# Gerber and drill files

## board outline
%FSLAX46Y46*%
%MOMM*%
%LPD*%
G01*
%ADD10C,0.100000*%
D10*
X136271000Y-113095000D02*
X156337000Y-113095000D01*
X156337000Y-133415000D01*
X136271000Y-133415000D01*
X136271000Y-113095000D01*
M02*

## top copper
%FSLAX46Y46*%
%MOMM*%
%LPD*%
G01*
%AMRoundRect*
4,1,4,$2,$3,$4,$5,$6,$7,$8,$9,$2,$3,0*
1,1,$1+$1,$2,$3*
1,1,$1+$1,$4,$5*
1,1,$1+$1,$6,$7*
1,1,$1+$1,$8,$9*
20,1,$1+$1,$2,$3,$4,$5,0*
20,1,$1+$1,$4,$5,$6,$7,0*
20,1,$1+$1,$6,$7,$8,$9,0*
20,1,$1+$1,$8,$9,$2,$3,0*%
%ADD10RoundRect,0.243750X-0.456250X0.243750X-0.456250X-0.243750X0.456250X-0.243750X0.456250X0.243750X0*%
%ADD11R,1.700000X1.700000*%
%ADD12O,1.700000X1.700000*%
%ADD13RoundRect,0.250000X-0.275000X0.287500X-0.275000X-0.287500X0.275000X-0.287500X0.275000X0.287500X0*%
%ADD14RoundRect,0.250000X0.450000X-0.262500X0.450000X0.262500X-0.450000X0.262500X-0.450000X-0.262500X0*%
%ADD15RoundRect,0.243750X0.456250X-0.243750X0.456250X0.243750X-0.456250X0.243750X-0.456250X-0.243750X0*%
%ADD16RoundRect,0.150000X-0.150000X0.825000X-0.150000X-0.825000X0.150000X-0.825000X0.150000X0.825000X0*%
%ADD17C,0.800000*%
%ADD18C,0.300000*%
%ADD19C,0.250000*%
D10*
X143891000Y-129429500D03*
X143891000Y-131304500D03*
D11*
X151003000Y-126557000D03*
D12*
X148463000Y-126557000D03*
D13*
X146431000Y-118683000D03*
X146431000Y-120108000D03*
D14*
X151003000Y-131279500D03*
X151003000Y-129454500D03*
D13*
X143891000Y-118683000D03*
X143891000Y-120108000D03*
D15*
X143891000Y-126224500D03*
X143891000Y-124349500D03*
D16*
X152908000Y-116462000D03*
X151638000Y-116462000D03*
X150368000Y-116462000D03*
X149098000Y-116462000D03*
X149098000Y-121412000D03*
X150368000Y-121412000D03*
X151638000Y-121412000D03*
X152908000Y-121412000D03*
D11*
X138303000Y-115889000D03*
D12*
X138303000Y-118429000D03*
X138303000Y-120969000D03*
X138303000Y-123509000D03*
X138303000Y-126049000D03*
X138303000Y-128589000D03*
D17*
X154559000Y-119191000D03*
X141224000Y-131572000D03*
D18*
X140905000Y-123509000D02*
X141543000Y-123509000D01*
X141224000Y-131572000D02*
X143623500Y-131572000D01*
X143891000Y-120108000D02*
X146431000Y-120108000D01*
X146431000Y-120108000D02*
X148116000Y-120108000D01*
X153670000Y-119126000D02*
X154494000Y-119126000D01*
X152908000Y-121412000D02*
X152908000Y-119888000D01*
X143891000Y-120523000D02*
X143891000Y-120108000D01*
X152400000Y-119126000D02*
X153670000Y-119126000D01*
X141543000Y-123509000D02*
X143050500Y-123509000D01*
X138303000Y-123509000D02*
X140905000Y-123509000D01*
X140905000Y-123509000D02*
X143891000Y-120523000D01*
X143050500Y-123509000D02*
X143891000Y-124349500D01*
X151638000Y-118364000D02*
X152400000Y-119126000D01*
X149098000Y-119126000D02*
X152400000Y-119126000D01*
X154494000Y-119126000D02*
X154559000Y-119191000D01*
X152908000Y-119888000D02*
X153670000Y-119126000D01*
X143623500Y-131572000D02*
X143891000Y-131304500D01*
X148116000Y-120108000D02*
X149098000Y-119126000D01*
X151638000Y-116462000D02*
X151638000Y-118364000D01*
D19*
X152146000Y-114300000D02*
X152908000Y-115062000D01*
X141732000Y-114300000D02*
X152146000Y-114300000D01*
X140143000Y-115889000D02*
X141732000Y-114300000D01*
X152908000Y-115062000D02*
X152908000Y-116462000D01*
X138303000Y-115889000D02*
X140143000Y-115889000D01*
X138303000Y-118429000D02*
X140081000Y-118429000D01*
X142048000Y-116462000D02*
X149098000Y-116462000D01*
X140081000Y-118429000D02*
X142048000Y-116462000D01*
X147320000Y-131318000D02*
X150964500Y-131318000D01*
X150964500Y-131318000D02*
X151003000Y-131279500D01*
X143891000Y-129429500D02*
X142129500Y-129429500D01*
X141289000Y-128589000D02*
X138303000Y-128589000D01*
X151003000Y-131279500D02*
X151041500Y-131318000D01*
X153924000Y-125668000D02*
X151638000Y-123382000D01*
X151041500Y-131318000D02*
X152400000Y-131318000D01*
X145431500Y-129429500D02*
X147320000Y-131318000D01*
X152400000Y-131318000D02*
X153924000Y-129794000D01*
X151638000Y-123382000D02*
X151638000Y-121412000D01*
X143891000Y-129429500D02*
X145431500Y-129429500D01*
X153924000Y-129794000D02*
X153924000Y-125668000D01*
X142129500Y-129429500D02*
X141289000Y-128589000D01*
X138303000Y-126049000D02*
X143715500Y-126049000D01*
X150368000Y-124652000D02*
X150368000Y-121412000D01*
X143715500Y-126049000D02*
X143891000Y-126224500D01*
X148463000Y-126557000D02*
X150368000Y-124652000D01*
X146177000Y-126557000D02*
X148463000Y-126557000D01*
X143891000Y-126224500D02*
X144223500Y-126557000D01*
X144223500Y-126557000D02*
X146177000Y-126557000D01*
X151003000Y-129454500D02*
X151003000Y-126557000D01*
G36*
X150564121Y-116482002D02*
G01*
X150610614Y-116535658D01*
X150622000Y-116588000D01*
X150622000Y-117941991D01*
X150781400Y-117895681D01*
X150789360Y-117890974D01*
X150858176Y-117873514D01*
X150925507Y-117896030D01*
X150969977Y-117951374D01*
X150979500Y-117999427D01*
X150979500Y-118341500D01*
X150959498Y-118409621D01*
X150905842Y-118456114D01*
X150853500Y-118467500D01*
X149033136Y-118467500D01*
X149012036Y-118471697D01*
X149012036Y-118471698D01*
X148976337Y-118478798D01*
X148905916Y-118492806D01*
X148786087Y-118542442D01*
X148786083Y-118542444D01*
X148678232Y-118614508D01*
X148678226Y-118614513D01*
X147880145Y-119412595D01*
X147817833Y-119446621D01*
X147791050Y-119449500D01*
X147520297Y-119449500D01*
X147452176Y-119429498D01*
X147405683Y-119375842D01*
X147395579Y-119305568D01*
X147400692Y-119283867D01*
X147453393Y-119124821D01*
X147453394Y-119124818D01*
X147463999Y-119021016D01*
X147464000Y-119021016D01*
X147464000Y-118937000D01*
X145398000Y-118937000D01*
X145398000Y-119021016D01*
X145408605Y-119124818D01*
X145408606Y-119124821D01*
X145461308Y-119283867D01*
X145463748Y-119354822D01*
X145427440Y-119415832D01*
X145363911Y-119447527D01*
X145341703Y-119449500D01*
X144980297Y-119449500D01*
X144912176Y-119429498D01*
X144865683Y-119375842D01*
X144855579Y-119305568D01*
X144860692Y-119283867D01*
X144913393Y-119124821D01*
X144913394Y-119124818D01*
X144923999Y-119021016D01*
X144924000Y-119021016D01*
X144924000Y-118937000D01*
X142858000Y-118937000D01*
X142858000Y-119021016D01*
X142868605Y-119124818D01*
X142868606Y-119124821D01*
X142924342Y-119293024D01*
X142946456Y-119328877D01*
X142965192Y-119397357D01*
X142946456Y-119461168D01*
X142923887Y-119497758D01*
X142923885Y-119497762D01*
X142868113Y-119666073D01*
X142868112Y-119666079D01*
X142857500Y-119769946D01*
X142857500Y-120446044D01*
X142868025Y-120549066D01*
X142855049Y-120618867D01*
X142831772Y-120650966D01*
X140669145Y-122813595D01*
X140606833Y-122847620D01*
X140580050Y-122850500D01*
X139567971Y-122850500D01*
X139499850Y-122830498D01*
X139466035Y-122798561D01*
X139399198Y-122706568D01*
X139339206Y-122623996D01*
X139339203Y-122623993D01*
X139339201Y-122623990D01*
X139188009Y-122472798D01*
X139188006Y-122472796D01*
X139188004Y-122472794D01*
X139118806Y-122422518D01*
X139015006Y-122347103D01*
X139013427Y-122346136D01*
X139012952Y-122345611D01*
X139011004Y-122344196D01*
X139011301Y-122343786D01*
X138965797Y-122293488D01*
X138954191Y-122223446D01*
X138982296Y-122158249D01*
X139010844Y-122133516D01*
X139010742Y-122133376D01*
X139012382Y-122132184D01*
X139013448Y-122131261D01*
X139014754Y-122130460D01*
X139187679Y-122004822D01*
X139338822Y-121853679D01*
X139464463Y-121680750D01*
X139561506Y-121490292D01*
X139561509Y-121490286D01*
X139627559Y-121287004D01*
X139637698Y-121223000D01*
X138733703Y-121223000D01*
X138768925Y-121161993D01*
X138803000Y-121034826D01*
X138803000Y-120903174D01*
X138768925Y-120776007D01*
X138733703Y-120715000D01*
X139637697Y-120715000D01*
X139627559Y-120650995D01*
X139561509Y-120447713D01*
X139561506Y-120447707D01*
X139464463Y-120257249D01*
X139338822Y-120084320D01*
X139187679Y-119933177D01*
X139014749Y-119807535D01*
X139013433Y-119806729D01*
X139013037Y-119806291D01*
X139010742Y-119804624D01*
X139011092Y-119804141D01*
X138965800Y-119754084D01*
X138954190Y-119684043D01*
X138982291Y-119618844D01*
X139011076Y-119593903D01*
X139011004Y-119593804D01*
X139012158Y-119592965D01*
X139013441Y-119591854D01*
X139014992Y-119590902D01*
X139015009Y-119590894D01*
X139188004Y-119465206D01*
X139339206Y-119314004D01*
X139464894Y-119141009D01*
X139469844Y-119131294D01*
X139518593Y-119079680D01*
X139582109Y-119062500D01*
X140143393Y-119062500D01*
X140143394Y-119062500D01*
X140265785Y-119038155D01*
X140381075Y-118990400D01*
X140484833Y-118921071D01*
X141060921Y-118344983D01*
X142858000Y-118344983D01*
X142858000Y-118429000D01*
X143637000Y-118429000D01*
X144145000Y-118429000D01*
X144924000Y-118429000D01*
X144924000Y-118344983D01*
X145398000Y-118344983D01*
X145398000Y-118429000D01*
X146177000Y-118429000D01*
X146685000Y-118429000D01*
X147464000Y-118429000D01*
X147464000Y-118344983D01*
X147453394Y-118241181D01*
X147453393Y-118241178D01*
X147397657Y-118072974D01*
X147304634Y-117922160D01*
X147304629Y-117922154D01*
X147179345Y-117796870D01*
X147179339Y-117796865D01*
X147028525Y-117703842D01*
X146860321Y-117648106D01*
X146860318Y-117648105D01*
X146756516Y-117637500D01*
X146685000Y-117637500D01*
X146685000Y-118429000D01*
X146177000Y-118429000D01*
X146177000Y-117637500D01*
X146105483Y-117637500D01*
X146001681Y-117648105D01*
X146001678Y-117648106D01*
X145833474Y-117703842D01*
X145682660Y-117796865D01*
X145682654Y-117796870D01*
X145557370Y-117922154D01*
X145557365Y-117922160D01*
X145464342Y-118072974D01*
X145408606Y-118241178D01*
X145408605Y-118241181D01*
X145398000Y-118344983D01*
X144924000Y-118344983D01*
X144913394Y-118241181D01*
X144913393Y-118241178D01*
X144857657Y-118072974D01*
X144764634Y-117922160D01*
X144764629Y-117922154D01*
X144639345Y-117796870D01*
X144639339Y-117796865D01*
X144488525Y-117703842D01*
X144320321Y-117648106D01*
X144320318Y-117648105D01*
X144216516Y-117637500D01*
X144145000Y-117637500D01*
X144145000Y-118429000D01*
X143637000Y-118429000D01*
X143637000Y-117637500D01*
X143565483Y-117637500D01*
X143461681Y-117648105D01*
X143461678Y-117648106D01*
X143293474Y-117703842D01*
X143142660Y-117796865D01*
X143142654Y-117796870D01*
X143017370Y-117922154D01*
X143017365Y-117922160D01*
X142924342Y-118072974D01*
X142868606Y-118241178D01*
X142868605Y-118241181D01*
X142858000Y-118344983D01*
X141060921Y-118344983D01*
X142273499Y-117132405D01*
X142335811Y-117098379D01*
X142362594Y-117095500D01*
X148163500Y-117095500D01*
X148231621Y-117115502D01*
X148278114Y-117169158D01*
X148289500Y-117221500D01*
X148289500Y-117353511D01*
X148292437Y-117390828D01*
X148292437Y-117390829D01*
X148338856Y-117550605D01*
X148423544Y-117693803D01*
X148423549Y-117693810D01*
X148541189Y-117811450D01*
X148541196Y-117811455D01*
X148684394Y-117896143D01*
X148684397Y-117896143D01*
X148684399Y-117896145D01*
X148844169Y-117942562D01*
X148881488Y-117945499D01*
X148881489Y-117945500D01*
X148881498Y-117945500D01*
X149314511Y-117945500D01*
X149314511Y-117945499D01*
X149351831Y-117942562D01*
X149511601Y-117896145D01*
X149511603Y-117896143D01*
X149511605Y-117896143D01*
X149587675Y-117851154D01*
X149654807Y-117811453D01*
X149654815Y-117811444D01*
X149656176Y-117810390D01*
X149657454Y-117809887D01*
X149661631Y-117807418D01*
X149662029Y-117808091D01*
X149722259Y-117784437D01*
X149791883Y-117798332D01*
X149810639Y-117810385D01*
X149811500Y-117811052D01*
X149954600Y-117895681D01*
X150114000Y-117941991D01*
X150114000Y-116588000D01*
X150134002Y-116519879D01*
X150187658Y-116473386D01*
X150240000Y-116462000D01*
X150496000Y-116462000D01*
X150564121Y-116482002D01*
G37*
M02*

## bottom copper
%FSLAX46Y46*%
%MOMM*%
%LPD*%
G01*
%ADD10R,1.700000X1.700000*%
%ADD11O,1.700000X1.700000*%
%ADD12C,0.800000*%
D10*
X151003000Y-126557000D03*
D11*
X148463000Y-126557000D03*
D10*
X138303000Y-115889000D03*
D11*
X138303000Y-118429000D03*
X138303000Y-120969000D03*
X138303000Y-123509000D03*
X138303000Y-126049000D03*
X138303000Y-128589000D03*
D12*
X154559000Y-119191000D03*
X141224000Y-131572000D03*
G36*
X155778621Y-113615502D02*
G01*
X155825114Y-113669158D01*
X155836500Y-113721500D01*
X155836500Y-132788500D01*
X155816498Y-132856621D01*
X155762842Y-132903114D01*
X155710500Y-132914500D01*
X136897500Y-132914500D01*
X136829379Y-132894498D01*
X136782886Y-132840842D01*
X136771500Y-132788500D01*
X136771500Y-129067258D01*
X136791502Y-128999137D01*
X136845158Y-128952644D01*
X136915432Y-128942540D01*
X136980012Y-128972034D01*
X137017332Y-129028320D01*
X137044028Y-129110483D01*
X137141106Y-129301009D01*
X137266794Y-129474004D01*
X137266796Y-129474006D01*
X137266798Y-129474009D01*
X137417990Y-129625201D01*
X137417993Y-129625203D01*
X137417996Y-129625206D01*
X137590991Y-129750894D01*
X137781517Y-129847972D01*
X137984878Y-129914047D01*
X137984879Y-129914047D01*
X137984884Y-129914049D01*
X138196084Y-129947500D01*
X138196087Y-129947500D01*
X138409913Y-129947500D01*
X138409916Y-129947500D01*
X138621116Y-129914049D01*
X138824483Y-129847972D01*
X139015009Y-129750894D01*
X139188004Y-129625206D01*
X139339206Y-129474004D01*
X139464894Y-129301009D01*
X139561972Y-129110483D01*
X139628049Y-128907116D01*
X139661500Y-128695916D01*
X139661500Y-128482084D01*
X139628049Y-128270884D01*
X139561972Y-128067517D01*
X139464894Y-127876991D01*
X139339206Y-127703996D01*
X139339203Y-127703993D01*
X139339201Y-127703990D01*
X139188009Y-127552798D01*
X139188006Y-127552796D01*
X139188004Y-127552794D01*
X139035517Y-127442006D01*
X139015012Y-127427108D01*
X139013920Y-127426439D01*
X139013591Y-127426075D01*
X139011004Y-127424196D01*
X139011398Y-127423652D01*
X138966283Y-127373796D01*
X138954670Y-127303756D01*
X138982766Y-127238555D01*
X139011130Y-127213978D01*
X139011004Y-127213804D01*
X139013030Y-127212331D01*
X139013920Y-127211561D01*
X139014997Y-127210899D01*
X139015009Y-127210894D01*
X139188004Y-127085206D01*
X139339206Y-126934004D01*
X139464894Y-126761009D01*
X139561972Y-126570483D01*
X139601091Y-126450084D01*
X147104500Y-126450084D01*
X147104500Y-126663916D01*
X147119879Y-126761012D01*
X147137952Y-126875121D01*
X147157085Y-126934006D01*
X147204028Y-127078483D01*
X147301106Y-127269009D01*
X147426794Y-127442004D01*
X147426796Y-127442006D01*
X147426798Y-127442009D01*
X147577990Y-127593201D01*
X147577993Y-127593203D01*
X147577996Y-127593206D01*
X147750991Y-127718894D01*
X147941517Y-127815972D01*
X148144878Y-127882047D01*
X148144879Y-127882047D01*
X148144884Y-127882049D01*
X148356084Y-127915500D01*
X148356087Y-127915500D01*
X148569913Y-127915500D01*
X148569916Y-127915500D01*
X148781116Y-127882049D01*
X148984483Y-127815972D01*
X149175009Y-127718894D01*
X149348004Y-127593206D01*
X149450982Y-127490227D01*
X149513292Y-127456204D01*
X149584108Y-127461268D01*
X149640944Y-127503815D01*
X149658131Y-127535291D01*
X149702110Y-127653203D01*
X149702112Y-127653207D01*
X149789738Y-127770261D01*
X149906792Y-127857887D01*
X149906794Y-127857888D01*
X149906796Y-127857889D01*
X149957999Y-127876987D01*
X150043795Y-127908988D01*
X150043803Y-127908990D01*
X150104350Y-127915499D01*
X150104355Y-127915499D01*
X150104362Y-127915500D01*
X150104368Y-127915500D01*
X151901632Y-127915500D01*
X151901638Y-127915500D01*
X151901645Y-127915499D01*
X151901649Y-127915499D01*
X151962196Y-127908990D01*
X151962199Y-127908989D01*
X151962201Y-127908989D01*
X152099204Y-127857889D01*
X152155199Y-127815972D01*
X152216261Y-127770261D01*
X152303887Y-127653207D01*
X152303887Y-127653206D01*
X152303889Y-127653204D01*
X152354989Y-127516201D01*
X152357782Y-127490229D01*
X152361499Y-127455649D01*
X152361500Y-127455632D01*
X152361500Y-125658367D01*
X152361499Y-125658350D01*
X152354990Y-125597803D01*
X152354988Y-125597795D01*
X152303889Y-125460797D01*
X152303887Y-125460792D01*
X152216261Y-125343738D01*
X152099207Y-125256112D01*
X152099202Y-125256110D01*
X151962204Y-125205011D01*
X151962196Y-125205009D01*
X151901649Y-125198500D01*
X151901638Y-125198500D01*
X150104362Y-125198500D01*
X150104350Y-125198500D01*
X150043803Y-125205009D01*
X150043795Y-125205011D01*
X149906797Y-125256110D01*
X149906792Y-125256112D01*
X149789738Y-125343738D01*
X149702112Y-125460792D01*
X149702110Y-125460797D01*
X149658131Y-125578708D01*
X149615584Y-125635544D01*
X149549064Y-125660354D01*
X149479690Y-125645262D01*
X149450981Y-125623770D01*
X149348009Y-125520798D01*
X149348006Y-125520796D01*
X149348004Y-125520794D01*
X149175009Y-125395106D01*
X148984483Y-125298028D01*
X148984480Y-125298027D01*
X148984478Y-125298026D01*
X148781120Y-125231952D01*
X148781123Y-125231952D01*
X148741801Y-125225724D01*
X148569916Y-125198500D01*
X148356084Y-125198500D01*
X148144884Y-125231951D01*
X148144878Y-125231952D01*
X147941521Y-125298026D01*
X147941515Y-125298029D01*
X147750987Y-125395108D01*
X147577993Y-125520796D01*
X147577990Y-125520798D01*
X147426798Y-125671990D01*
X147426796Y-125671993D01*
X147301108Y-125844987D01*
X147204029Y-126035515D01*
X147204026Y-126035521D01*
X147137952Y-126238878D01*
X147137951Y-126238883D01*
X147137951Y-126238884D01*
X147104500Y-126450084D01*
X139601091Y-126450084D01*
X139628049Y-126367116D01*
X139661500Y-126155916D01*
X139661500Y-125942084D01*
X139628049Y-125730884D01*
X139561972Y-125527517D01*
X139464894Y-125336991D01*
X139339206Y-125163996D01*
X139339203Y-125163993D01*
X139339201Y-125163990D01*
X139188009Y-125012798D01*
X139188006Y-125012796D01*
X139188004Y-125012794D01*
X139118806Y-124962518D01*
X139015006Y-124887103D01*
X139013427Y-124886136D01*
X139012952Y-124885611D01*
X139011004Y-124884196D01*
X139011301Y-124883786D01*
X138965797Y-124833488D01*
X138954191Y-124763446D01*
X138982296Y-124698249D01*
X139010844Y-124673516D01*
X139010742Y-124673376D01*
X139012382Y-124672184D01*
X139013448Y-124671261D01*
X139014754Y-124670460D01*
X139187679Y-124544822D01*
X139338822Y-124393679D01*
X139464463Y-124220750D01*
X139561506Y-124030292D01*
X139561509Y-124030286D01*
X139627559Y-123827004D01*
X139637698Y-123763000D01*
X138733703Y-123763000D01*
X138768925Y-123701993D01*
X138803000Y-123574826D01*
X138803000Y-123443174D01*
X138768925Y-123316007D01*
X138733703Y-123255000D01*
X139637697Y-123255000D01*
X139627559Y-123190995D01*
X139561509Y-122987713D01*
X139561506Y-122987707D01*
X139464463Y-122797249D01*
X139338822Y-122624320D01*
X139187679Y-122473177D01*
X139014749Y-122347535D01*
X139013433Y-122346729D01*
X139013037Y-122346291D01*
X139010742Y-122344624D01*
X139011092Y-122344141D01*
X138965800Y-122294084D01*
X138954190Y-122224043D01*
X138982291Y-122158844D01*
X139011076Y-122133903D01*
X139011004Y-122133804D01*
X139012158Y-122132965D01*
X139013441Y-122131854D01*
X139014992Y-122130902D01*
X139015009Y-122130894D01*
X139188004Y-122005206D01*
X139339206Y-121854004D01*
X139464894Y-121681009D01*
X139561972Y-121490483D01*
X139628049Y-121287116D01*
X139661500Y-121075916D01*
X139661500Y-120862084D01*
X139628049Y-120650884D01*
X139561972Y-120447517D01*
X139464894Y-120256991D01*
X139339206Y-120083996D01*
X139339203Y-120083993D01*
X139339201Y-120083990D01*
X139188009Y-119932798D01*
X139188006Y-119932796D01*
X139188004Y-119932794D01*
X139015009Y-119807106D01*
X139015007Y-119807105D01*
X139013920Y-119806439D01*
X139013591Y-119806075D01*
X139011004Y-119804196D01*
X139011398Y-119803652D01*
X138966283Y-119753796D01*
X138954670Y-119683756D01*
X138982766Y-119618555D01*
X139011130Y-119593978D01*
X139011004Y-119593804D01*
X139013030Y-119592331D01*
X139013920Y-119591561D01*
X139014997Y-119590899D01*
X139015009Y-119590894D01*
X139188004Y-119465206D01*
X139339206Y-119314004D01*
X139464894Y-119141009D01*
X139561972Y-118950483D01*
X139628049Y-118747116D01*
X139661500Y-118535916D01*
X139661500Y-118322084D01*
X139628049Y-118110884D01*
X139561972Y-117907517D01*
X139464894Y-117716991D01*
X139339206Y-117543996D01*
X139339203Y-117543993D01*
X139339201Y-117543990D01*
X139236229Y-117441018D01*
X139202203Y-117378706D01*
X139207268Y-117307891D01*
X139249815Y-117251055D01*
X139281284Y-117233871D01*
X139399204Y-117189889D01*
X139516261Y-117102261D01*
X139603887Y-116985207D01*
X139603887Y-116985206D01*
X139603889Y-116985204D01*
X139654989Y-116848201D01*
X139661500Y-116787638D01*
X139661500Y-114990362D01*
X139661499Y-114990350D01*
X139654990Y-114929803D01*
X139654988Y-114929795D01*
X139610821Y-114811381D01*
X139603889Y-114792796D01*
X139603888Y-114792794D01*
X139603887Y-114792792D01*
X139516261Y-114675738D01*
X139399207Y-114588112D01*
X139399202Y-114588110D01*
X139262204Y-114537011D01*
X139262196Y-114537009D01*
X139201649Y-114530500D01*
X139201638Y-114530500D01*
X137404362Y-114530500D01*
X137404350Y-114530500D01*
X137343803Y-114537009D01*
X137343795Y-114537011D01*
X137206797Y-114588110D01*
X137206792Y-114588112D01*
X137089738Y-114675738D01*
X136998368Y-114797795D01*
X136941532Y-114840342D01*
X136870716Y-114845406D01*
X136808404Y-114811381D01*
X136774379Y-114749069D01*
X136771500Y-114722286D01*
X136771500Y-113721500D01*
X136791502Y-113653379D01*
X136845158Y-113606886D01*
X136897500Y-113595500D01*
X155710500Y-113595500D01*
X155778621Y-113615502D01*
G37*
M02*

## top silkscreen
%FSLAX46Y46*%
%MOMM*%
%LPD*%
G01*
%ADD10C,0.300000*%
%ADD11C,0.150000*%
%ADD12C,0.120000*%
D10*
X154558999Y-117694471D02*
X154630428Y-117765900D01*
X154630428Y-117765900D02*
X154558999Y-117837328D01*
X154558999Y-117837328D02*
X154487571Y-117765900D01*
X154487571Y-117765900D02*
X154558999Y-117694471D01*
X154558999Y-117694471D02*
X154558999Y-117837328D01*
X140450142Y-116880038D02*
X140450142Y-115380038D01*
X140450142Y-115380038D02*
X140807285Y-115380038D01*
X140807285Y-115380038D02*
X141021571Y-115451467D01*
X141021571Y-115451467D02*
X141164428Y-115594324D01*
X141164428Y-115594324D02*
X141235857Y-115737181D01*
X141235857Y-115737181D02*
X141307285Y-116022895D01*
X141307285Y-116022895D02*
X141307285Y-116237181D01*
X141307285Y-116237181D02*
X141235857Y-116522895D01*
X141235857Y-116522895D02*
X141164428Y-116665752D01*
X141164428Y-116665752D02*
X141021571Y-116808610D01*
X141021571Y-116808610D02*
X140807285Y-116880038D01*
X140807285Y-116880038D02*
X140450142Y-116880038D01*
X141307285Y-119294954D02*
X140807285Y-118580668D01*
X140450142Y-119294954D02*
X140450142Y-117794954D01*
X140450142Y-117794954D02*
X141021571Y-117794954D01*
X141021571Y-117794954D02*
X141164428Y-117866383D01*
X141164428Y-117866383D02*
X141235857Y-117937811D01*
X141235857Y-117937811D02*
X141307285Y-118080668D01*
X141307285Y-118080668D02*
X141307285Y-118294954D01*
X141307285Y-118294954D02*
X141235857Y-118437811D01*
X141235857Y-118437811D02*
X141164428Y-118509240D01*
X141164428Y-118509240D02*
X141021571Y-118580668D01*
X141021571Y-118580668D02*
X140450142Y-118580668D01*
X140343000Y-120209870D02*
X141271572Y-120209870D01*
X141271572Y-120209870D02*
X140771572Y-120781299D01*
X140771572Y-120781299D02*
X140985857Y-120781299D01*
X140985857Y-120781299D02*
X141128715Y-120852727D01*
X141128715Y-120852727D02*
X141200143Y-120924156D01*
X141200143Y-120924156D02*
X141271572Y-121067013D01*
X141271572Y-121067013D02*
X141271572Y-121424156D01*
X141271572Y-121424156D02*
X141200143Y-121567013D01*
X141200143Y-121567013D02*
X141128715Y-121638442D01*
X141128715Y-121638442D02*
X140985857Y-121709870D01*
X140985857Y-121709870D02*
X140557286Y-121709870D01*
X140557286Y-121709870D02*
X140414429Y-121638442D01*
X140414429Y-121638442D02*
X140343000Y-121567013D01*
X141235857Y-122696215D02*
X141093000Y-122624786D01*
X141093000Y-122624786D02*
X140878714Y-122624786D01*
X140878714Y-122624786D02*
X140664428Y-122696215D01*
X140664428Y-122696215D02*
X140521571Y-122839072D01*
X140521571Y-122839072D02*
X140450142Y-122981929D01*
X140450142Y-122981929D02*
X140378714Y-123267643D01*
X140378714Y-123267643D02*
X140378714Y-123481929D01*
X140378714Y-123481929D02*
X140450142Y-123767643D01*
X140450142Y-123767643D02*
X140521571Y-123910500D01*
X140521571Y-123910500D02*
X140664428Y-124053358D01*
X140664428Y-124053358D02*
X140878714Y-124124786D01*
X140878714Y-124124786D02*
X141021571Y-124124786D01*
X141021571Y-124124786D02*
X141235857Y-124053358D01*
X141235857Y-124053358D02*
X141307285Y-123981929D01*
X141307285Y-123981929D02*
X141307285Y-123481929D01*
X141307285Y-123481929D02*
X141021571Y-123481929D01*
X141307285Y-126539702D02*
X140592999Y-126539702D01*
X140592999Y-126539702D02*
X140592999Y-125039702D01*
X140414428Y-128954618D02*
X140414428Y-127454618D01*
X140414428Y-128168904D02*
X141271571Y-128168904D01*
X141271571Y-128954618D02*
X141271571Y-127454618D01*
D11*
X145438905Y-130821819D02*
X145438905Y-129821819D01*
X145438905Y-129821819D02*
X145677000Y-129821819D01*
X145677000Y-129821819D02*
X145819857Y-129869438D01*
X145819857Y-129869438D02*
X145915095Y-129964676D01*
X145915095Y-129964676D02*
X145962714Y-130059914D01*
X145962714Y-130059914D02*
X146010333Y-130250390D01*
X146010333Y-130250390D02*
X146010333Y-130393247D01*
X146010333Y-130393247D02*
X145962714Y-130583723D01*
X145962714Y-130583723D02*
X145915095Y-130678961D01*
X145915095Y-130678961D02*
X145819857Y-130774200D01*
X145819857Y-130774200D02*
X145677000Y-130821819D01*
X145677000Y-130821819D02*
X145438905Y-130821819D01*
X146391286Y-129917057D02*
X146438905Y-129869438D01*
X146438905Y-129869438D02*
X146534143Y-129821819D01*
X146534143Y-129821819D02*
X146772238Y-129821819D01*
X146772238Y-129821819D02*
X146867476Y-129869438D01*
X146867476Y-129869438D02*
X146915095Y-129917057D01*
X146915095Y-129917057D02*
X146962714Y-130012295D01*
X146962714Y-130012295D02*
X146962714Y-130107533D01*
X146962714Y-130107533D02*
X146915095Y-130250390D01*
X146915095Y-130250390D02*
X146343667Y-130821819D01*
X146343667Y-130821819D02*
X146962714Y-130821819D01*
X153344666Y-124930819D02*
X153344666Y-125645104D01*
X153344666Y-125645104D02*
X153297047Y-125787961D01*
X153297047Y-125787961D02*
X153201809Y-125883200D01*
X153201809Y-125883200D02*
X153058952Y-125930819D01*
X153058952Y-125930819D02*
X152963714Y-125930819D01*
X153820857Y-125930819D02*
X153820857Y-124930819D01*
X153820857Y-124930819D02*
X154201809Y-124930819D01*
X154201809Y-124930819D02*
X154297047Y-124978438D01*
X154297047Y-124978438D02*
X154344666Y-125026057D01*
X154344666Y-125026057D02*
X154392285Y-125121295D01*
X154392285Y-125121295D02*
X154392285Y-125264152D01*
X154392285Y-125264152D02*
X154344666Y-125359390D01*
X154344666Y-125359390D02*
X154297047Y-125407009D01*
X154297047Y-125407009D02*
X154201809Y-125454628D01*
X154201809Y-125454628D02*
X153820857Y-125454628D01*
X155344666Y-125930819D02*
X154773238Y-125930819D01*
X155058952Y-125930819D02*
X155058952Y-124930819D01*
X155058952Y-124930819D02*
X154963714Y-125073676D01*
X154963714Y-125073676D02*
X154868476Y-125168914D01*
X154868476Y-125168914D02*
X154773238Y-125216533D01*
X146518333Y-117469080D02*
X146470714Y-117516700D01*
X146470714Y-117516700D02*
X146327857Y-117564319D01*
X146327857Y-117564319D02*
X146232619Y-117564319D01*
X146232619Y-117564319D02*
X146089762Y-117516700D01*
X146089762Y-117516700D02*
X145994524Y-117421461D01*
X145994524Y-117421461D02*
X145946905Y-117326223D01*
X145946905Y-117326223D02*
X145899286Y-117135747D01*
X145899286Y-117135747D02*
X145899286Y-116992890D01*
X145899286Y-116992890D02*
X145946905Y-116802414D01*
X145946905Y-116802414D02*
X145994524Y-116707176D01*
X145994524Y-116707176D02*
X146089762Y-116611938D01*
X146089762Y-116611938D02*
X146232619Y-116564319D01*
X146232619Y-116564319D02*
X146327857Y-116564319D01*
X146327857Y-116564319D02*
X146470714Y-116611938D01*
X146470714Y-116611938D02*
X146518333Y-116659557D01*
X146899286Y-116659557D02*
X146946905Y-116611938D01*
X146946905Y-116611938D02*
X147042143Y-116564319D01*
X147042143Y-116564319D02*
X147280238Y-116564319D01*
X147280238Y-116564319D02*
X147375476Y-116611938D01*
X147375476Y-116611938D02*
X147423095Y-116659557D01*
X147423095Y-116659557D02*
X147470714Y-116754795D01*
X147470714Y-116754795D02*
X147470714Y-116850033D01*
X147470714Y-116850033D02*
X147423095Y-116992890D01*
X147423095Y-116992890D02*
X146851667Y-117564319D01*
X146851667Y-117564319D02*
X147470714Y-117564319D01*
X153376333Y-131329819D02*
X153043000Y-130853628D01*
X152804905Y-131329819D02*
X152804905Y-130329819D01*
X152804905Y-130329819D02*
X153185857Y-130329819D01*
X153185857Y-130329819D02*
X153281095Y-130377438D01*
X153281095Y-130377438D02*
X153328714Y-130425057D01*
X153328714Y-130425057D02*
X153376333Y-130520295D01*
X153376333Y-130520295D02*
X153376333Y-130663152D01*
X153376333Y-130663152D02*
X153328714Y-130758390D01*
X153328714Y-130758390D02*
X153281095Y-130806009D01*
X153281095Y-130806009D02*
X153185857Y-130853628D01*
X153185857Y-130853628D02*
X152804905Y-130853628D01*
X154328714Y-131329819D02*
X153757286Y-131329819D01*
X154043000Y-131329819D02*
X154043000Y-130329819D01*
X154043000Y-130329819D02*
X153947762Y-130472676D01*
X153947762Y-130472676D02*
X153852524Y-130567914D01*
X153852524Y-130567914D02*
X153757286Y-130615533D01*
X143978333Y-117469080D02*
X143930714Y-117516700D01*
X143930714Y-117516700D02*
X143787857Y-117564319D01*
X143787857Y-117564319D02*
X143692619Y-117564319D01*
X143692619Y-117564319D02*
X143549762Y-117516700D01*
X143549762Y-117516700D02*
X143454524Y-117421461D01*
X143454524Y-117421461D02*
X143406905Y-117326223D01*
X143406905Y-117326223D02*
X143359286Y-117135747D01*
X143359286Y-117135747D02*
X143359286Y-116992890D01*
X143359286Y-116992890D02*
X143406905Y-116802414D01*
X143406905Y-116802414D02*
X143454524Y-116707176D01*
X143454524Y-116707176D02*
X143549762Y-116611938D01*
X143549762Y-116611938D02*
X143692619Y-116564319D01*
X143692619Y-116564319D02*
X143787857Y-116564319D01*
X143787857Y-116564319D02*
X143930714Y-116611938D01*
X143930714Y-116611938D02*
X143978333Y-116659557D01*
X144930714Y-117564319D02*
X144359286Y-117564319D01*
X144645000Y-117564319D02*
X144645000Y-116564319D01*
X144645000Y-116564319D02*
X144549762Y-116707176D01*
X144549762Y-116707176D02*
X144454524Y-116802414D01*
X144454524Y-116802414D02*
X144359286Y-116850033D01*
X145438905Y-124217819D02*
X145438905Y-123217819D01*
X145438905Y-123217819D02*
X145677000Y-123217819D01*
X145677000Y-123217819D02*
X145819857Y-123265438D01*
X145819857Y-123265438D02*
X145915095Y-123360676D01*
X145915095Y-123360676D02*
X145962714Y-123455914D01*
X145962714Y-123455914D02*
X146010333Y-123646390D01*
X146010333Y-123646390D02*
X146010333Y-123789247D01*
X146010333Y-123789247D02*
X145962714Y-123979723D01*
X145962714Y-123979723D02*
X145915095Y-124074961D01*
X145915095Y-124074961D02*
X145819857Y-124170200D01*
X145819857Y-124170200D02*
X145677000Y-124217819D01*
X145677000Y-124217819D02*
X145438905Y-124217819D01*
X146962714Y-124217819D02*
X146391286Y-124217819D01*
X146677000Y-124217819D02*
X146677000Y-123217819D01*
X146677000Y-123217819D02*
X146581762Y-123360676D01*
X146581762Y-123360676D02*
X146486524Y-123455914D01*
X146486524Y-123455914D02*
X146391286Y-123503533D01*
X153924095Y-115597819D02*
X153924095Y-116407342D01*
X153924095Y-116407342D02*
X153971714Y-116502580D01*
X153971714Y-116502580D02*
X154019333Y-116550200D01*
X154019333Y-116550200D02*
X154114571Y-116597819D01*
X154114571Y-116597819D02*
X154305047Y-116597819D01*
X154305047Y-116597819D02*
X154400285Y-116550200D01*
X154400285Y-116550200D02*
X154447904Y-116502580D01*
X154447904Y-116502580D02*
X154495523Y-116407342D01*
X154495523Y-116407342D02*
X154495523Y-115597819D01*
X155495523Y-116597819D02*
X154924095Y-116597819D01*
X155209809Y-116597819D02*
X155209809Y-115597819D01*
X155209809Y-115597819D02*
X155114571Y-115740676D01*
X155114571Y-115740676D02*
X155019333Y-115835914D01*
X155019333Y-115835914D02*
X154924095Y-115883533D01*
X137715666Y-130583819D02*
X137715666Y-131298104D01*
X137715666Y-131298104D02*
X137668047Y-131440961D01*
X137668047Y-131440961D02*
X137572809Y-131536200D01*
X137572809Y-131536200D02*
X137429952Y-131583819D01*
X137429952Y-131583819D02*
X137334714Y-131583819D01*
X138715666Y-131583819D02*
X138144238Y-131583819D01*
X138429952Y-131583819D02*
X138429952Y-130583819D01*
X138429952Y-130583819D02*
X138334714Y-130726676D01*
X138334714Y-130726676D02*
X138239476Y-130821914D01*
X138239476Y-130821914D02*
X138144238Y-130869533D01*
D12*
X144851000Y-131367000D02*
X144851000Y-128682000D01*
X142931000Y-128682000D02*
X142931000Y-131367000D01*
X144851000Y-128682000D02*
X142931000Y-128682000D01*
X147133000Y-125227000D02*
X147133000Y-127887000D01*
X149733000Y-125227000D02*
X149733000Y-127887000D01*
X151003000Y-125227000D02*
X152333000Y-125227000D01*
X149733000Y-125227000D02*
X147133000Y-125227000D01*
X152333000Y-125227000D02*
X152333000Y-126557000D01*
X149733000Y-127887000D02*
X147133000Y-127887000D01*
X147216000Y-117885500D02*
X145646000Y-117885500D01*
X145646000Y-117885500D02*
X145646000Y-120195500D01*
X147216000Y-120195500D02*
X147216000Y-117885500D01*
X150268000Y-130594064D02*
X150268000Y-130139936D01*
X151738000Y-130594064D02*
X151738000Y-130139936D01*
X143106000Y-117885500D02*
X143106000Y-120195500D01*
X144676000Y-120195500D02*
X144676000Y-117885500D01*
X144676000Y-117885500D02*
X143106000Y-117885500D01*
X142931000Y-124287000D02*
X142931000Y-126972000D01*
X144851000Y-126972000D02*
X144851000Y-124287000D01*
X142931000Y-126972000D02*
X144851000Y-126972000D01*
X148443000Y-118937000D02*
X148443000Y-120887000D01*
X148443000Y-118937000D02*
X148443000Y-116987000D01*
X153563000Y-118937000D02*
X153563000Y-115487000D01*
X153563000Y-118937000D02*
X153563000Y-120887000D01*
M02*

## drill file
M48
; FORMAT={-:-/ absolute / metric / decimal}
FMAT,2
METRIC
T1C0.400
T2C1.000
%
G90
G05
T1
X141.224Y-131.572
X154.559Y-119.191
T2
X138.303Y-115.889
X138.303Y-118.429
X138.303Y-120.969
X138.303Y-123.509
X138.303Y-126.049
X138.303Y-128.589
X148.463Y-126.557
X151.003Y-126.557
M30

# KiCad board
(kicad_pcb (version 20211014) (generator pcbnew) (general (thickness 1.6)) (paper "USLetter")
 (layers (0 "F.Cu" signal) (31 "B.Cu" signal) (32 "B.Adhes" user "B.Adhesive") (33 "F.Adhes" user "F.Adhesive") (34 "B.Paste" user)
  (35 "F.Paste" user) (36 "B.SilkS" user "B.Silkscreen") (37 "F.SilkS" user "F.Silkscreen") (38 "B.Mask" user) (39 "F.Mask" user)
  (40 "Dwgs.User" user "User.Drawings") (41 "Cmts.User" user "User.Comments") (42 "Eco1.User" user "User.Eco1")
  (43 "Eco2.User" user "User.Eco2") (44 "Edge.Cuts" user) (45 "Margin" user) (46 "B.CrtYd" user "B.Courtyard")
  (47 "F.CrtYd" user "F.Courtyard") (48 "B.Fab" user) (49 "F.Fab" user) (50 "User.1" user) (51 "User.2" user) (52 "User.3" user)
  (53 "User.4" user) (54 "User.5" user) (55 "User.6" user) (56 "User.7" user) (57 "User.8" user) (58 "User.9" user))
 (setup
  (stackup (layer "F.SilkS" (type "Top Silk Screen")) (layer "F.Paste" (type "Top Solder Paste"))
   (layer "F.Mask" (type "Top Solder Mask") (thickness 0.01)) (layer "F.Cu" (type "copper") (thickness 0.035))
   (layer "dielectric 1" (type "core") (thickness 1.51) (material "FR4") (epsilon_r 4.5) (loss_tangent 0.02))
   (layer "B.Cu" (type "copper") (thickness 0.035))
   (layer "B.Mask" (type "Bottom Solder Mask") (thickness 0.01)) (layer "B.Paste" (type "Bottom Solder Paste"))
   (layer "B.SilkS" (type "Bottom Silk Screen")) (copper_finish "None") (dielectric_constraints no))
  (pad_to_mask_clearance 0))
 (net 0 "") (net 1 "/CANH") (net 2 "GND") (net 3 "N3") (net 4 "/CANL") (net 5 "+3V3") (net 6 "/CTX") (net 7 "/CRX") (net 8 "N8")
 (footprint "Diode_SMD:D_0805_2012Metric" (layer "F.Cu") (at 143.891 130.367 -90)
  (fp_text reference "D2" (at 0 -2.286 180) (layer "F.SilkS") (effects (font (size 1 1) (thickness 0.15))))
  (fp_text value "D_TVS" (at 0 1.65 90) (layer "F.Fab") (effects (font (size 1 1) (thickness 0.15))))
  (fp_line (start 1 -0.96) (end -1.685 -0.96) (layer "F.SilkS") (width 0.12))
  (fp_line (start -1.685 0.96) (end 1 0.96) (layer "F.SilkS") (width 0.12))
  (fp_line (start -1.685 -0.96) (end -1.685 0.96) (layer "F.SilkS") (width 0.12))
  (pad "1" smd roundrect (at -0.9375 0 270) (size 0.975 1.4) (layers "F.Cu" "F.Paste" "F.Mask") (roundrect_rratio 0.25) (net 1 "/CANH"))
  (pad "2" smd roundrect (at 0.9375 0 270) (size 0.975 1.4) (layers "F.Cu" "F.Paste" "F.Mask") (roundrect_rratio 0.25) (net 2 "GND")))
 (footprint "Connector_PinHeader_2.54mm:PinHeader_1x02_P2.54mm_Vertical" (layer "F.Cu") (at 151.003 126.557 -90)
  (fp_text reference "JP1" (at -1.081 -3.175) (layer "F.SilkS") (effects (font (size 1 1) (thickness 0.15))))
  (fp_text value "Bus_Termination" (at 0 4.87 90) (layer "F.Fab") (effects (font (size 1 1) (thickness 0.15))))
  (fp_line (start -1.33 3.87) (end 1.33 3.87) (layer "F.SilkS") (width 0.12))
  (fp_line (start -1.33 1.27) (end 1.33 1.27) (layer "F.SilkS") (width 0.12))
  (fp_line (start -1.33 0) (end -1.33 -1.33) (layer "F.SilkS") (width 0.12))
  (fp_line (start -1.33 1.27) (end -1.33 3.87) (layer "F.SilkS") (width 0.12))
  (fp_line (start -1.33 -1.33) (end 0 -1.33) (layer "F.SilkS") (width 0.12))
  (fp_line (start 1.33 1.27) (end 1.33 3.87) (layer "F.SilkS") (width 0.12))
  (pad "1" thru_hole rect (at 0 0 270) (size 1.7 1.7) (drill 1) (layers *.Cu *.Mask) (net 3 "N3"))
  (pad "2" thru_hole oval (at 0 2.54 270) (size 1.7 1.7) (drill 1) (layers *.Cu *.Mask) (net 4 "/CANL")))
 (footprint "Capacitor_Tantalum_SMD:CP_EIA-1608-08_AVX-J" (layer "F.Cu") (at 146.431 119.3955 -90)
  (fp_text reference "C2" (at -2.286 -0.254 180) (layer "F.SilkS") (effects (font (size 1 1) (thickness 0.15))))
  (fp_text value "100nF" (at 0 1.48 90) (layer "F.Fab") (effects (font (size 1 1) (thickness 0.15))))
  (fp_line (start -1.51 -0.785) (end -1.51 0.785) (layer "F.SilkS") (width 0.12))
  (fp_line (start -1.51 0.785) (end 0.8 0.785) (layer "F.SilkS") (width 0.12))
  (fp_line (start 0.8 -0.785) (end -1.51 -0.785) (layer "F.SilkS") (width 0.12))
  (pad "1" smd roundrect (at -0.7125 0 270) (size 1.075 1.05) (layers "F.Cu" "F.Paste" "F.Mask") (roundrect_rratio 0.238095) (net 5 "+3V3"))
  (pad "2" smd roundrect (at 0.7125 0 270) (size 1.075 1.05) (layers "F.Cu" "F.Paste" "F.Mask") (roundrect_rratio 0.238095) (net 2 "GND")))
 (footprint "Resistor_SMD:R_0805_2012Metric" (layer "F.Cu") (at 151.003 130.367 90)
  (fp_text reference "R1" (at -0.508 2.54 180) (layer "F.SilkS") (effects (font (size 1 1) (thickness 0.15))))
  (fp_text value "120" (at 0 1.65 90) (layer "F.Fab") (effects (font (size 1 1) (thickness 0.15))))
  (fp_line (start -0.227064 -0.735) (end 0.227064 -0.735) (layer "F.SilkS") (width 0.12))
  (fp_line (start -0.227064 0.735) (end 0.227064 0.735) (layer "F.SilkS") (width 0.12))
  (pad "1" smd roundrect (at -0.9125 0 90) (size 1.025 1.4) (layers "F.Cu" "F.Paste" "F.Mask") (roundrect_rratio 0.243902) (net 1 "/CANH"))
  (pad "2" smd roundrect (at 0.9125 0 90) (size 1.025 1.4) (layers "F.Cu" "F.Paste" "F.Mask") (roundrect_rratio 0.243902) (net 3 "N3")))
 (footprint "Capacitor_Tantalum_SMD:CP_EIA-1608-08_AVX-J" (layer "F.Cu") (at 143.891 119.3955 -90)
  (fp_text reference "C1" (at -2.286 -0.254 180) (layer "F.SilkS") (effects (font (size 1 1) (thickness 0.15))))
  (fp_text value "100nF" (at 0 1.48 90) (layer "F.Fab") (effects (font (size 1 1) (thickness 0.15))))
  (fp_line (start -1.51 0.785) (end 0.8 0.785) (layer "F.SilkS") (width 0.12))
  (fp_line (start 0.8 -0.785) (end -1.51 -0.785) (layer "F.SilkS") (width 0.12))
  (fp_line (start -1.51 -0.785) (end -1.51 0.785) (layer "F.SilkS") (width 0.12))
  (pad "1" smd roundrect (at -0.7125 0 270) (size 1.075 1.05) (layers "F.Cu" "F.Paste" "F.Mask") (roundrect_rratio 0.238095) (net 5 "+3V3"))
  (pad "2" smd roundrect (at 0.7125 0 270) (size 1.075 1.05) (layers "F.Cu" "F.Paste" "F.Mask") (roundrect_rratio 0.238095) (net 2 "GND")))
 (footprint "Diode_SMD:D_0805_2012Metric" (layer "F.Cu") (at 143.891 125.287 90)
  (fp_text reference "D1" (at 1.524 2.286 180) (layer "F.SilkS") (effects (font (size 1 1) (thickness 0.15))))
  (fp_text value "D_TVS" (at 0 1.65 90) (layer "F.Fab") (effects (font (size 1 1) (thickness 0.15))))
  (fp_line (start 1 -0.96) (end -1.685 -0.96) (layer "F.SilkS") (width 0.12))
  (fp_line (start -1.685 0.96) (end 1 0.96) (layer "F.SilkS") (width 0.12))
  (fp_line (start -1.685 -0.96) (end -1.685 0.96) (layer "F.SilkS") (width 0.12))
  (pad "1" smd roundrect (at -0.9375 0 90) (size 0.975 1.4) (layers "F.Cu" "F.Paste" "F.Mask") (roundrect_rratio 0.25) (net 4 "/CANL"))
  (pad "2" smd roundrect (at 0.9375 0 90) (size 0.975 1.4) (layers "F.Cu" "F.Paste" "F.Mask") (roundrect_rratio 0.25) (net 2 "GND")))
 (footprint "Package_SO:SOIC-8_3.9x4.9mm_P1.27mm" (layer "F.Cu") (at 151.003 118.937 -90)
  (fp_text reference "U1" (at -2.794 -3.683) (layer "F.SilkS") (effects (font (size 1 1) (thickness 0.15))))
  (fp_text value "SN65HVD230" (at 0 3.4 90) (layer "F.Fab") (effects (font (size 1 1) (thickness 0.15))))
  (fp_line (start 0 2.56) (end 1.95 2.56) (layer "F.SilkS") (width 0.12))
  (fp_line (start 0 2.56) (end -1.95 2.56) (layer "F.SilkS") (width 0.12))
  (fp_line (start 0 -2.56) (end -3.45 -2.56) (layer "F.SilkS") (width 0.12))
  (fp_line (start 0 -2.56) (end 1.95 -2.56) (layer "F.SilkS") (width 0.12))
  (pad "1" smd roundrect (at -2.475 -1.905 270) (size 1.95 0.6) (layers "F.Cu" "F.Paste" "F.Mask") (roundrect_rratio 0.25) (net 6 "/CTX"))
  (pad "2" smd roundrect (at -2.475 -0.635 270) (size 1.95 0.6) (layers "F.Cu" "F.Paste" "F.Mask") (roundrect_rratio 0.25) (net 2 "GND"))
  (pad "3" smd roundrect (at -2.475 0.635 270) (size 1.95 0.6) (layers "F.Cu" "F.Paste" "F.Mask") (roundrect_rratio 0.25) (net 5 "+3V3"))
  (pad "4" smd roundrect (at -2.475 1.905 270) (size 1.95 0.6) (layers "F.Cu" "F.Paste" "F.Mask") (roundrect_rratio 0.25) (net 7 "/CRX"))
  (pad "5" smd roundrect (at 2.475 1.905 270) (size 1.95 0.6) (layers "F.Cu" "F.Paste" "F.Mask") (roundrect_rratio 0.25) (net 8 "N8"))
  (pad "6" smd roundrect (at 2.475 0.635 270) (size 1.95 0.6) (layers "F.Cu" "F.Paste" "F.Mask") (roundrect_rratio 0.25) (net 4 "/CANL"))
  (pad "7" smd roundrect (at 2.475 -0.635 270) (size 1.95 0.6) (layers "F.Cu" "F.Paste" "F.Mask") (roundrect_rratio 0.25) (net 1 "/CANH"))
  (pad "8" smd roundrect (at 2.475 -1.905 270) (size 1.95 0.6) (layers "F.Cu" "F.Paste" "F.Mask") (roundrect_rratio 0.25) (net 2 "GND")))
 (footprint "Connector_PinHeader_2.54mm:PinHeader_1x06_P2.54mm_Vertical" (layer "B.Cu") (at 138.303 115.889 180)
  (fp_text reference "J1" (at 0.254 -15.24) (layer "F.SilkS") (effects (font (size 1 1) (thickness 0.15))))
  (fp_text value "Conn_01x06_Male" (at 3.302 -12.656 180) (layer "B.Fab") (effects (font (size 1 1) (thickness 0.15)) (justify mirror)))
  (pad "1" thru_hole rect (at 0 0 180) (size 1.7 1.7) (drill 1) (layers *.Cu *.Mask) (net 6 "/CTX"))
  (pad "2" thru_hole oval (at 0 -2.54 180) (size 1.7 1.7) (drill 1) (layers *.Cu *.Mask) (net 7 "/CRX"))
  (pad "3" thru_hole oval (at 0 -5.08 180) (size 1.7 1.7) (drill 1) (layers *.Cu *.Mask) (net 5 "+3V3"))
  (pad "4" thru_hole oval (at 0 -7.62 180) (size 1.7 1.7) (drill 1) (layers *.Cu *.Mask) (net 2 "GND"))
  (pad "5" thru_hole oval (at 0 -10.16 180) (size 1.7 1.7) (drill 1) (layers *.Cu *.Mask) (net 4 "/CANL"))
  (pad "6" thru_hole oval (at 0 -12.7 180) (size 1.7 1.7) (drill 1) (layers *.Cu *.Mask) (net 1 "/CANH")))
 (gr_rect (start 136.271 113.095) (end 156.337 133.415) (layer "Edge.Cuts") (width 0.1) (fill none))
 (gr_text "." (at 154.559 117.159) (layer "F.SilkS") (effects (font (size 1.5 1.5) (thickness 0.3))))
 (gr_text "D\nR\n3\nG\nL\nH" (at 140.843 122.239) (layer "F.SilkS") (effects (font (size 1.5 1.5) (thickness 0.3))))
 (segment (start 140.905 123.509) (end 141.543 123.509) (width 0.3) (layer "F.Cu") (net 2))
 (segment (start 141.224 131.572) (end 143.6235 131.572) (width 0.3) (layer "F.Cu") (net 2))
 (segment (start 143.891 120.108) (end 146.431 120.108) (width 0.3) (layer "F.Cu") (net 2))
 (segment (start 146.431 120.108) (end 148.116 120.108) (width 0.3) (layer "F.Cu") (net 2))
 (segment (start 153.67 119.126) (end 154.494 119.126) (width 0.3) (layer "F.Cu") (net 2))
 (segment (start 152.908 121.412) (end 152.908 119.888) (width 0.3) (layer "F.Cu") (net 2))
 (segment (start 143.891 120.523) (end 143.891 120.108) (width 0.3) (layer "F.Cu") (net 2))
 (segment (start 152.4 119.126) (end 153.67 119.126) (width 0.3) (layer "F.Cu") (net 2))
 (segment (start 141.543 123.509) (end 143.0505 123.509) (width 0.3) (layer "F.Cu") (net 2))
 (segment (start 138.303 123.509) (end 140.905 123.509) (width 0.3) (layer "F.Cu") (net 2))
 (segment (start 140.905 123.509) (end 143.891 120.523) (width 0.3) (layer "F.Cu") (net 2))
 (segment (start 143.0505 123.509) (end 143.891 124.3495) (width 0.3) (layer "F.Cu") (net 2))
 (segment (start 151.638 118.364) (end 152.4 119.126) (width 0.3) (layer "F.Cu") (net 2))
 (segment (start 149.098 119.126) (end 152.4 119.126) (width 0.3) (layer "F.Cu") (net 2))
 (segment (start 154.494 119.126) (end 154.559 119.191) (width 0.3) (layer "F.Cu") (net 2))
 (segment (start 152.908 119.888) (end 153.67 119.126) (width 0.3) (layer "F.Cu") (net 2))
 (segment (start 143.6235 131.572) (end 143.891 131.3045) (width 0.3) (layer "F.Cu") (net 2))
 (segment (start 148.116 120.108) (end 149.098 119.126) (width 0.3) (layer "F.Cu") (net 2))
 (segment (start 151.638 116.462) (end 151.638 118.364) (width 0.3) (layer "F.Cu") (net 2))
 (via (at 154.559 119.191) (size 0.8) (drill 0.4) (layers "F.Cu" "B.Cu") (free) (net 2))
 (via (at 141.224 131.572) (size 0.8) (drill 0.4) (layers "F.Cu" "B.Cu") (free) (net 2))
 (segment (start 152.146 114.3) (end 152.908 115.062) (width 0.25) (layer "F.Cu") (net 6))
 (segment (start 141.732 114.3) (end 152.146 114.3) (width 0.25) (layer "F.Cu") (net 6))
 (segment (start 140.143 115.889) (end 141.732 114.3) (width 0.25) (layer "F.Cu") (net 6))
 (segment (start 152.908 115.062) (end 152.908 116.462) (width 0.25) (layer "F.Cu") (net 6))
 (segment (start 138.303 115.889) (end 140.143 115.889) (width 0.25) (layer "F.Cu") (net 6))
 (segment (start 138.303 118.429) (end 140.081 118.429) (width 0.25) (layer "F.Cu") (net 7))
 (segment (start 142.048 116.462) (end 149.098 116.462) (width 0.25) (layer "F.Cu") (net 7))
 (segment (start 140.081 118.429) (end 142.048 116.462) (width 0.25) (layer "F.Cu") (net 7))
 (segment (start 147.32 131.318) (end 150.9645 131.318) (width 0.25) (layer "F.Cu") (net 1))
 (segment (start 150.9645 131.318) (end 151.003 131.2795) (width 0.25) (layer "F.Cu") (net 1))
 (segment (start 143.891 129.4295) (end 142.1295 129.4295) (width 0.25) (layer "F.Cu") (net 1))
 (segment (start 141.289 128.589) (end 138.303 128.589) (width 0.25) (layer "F.Cu") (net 1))
 (segment (start 151.003 131.2795) (end 151.0415 131.318) (width 0.25) (layer "F.Cu") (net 1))
 (segment (start 153.924 125.668) (end 151.638 123.382) (width 0.25) (layer "F.Cu") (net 1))
 (segment (start 151.0415 131.318) (end 152.4 131.318) (width 0.25) (layer "F.Cu") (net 1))
 (segment (start 145.4315 129.4295) (end 147.32 131.318) (width 0.25) (layer "F.Cu") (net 1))
 (segment (start 152.4 131.318) (end 153.924 129.794) (width 0.25) (layer "F.Cu") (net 1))
 (segment (start 151.638 123.382) (end 151.638 121.412) (width 0.25) (layer "F.Cu") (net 1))
 (segment (start 143.891 129.4295) (end 145.4315 129.4295) (width 0.25) (layer "F.Cu") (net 1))
 (segment (start 153.924 129.794) (end 153.924 125.668) (width 0.25) (layer "F.Cu") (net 1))
 (segment (start 142.1295 129.4295) (end 141.289 128.589) (width 0.25) (layer "F.Cu") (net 1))
 (segment (start 138.303 126.049) (end 143.7155 126.049) (width 0.25) (layer "F.Cu") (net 4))
 (segment (start 150.368 124.652) (end 150.368 121.412) (width 0.25) (layer "F.Cu") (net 4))
 (segment (start 143.7155 126.049) (end 143.891 126.2245) (width 0.25) (layer "F.Cu") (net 4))
 (segment (start 148.463 126.557) (end 150.368 124.652) (width 0.25) (layer "F.Cu") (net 4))
 (segment (start 146.177 126.557) (end 148.463 126.557) (width 0.25) (layer "F.Cu") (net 4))
 (segment (start 143.891 126.2245) (end 144.2235 126.557) (width 0.25) (layer "F.Cu") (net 4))
 (segment (start 144.2235 126.557) (end 146.177 126.557) (width 0.25) (layer "F.Cu") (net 4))
 (segment (start 151.003 129.4545) (end 151.003 126.557) (width 0.25) (layer "F.Cu") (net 3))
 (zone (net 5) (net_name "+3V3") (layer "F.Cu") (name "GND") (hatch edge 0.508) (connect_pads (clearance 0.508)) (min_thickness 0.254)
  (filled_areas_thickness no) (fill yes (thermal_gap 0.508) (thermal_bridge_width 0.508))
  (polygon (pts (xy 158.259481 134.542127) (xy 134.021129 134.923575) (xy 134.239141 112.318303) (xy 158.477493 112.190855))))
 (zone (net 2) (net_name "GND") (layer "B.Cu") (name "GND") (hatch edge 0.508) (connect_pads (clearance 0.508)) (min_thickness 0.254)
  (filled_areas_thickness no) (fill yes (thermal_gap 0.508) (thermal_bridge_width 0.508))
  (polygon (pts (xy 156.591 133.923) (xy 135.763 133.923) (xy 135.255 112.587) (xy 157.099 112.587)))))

